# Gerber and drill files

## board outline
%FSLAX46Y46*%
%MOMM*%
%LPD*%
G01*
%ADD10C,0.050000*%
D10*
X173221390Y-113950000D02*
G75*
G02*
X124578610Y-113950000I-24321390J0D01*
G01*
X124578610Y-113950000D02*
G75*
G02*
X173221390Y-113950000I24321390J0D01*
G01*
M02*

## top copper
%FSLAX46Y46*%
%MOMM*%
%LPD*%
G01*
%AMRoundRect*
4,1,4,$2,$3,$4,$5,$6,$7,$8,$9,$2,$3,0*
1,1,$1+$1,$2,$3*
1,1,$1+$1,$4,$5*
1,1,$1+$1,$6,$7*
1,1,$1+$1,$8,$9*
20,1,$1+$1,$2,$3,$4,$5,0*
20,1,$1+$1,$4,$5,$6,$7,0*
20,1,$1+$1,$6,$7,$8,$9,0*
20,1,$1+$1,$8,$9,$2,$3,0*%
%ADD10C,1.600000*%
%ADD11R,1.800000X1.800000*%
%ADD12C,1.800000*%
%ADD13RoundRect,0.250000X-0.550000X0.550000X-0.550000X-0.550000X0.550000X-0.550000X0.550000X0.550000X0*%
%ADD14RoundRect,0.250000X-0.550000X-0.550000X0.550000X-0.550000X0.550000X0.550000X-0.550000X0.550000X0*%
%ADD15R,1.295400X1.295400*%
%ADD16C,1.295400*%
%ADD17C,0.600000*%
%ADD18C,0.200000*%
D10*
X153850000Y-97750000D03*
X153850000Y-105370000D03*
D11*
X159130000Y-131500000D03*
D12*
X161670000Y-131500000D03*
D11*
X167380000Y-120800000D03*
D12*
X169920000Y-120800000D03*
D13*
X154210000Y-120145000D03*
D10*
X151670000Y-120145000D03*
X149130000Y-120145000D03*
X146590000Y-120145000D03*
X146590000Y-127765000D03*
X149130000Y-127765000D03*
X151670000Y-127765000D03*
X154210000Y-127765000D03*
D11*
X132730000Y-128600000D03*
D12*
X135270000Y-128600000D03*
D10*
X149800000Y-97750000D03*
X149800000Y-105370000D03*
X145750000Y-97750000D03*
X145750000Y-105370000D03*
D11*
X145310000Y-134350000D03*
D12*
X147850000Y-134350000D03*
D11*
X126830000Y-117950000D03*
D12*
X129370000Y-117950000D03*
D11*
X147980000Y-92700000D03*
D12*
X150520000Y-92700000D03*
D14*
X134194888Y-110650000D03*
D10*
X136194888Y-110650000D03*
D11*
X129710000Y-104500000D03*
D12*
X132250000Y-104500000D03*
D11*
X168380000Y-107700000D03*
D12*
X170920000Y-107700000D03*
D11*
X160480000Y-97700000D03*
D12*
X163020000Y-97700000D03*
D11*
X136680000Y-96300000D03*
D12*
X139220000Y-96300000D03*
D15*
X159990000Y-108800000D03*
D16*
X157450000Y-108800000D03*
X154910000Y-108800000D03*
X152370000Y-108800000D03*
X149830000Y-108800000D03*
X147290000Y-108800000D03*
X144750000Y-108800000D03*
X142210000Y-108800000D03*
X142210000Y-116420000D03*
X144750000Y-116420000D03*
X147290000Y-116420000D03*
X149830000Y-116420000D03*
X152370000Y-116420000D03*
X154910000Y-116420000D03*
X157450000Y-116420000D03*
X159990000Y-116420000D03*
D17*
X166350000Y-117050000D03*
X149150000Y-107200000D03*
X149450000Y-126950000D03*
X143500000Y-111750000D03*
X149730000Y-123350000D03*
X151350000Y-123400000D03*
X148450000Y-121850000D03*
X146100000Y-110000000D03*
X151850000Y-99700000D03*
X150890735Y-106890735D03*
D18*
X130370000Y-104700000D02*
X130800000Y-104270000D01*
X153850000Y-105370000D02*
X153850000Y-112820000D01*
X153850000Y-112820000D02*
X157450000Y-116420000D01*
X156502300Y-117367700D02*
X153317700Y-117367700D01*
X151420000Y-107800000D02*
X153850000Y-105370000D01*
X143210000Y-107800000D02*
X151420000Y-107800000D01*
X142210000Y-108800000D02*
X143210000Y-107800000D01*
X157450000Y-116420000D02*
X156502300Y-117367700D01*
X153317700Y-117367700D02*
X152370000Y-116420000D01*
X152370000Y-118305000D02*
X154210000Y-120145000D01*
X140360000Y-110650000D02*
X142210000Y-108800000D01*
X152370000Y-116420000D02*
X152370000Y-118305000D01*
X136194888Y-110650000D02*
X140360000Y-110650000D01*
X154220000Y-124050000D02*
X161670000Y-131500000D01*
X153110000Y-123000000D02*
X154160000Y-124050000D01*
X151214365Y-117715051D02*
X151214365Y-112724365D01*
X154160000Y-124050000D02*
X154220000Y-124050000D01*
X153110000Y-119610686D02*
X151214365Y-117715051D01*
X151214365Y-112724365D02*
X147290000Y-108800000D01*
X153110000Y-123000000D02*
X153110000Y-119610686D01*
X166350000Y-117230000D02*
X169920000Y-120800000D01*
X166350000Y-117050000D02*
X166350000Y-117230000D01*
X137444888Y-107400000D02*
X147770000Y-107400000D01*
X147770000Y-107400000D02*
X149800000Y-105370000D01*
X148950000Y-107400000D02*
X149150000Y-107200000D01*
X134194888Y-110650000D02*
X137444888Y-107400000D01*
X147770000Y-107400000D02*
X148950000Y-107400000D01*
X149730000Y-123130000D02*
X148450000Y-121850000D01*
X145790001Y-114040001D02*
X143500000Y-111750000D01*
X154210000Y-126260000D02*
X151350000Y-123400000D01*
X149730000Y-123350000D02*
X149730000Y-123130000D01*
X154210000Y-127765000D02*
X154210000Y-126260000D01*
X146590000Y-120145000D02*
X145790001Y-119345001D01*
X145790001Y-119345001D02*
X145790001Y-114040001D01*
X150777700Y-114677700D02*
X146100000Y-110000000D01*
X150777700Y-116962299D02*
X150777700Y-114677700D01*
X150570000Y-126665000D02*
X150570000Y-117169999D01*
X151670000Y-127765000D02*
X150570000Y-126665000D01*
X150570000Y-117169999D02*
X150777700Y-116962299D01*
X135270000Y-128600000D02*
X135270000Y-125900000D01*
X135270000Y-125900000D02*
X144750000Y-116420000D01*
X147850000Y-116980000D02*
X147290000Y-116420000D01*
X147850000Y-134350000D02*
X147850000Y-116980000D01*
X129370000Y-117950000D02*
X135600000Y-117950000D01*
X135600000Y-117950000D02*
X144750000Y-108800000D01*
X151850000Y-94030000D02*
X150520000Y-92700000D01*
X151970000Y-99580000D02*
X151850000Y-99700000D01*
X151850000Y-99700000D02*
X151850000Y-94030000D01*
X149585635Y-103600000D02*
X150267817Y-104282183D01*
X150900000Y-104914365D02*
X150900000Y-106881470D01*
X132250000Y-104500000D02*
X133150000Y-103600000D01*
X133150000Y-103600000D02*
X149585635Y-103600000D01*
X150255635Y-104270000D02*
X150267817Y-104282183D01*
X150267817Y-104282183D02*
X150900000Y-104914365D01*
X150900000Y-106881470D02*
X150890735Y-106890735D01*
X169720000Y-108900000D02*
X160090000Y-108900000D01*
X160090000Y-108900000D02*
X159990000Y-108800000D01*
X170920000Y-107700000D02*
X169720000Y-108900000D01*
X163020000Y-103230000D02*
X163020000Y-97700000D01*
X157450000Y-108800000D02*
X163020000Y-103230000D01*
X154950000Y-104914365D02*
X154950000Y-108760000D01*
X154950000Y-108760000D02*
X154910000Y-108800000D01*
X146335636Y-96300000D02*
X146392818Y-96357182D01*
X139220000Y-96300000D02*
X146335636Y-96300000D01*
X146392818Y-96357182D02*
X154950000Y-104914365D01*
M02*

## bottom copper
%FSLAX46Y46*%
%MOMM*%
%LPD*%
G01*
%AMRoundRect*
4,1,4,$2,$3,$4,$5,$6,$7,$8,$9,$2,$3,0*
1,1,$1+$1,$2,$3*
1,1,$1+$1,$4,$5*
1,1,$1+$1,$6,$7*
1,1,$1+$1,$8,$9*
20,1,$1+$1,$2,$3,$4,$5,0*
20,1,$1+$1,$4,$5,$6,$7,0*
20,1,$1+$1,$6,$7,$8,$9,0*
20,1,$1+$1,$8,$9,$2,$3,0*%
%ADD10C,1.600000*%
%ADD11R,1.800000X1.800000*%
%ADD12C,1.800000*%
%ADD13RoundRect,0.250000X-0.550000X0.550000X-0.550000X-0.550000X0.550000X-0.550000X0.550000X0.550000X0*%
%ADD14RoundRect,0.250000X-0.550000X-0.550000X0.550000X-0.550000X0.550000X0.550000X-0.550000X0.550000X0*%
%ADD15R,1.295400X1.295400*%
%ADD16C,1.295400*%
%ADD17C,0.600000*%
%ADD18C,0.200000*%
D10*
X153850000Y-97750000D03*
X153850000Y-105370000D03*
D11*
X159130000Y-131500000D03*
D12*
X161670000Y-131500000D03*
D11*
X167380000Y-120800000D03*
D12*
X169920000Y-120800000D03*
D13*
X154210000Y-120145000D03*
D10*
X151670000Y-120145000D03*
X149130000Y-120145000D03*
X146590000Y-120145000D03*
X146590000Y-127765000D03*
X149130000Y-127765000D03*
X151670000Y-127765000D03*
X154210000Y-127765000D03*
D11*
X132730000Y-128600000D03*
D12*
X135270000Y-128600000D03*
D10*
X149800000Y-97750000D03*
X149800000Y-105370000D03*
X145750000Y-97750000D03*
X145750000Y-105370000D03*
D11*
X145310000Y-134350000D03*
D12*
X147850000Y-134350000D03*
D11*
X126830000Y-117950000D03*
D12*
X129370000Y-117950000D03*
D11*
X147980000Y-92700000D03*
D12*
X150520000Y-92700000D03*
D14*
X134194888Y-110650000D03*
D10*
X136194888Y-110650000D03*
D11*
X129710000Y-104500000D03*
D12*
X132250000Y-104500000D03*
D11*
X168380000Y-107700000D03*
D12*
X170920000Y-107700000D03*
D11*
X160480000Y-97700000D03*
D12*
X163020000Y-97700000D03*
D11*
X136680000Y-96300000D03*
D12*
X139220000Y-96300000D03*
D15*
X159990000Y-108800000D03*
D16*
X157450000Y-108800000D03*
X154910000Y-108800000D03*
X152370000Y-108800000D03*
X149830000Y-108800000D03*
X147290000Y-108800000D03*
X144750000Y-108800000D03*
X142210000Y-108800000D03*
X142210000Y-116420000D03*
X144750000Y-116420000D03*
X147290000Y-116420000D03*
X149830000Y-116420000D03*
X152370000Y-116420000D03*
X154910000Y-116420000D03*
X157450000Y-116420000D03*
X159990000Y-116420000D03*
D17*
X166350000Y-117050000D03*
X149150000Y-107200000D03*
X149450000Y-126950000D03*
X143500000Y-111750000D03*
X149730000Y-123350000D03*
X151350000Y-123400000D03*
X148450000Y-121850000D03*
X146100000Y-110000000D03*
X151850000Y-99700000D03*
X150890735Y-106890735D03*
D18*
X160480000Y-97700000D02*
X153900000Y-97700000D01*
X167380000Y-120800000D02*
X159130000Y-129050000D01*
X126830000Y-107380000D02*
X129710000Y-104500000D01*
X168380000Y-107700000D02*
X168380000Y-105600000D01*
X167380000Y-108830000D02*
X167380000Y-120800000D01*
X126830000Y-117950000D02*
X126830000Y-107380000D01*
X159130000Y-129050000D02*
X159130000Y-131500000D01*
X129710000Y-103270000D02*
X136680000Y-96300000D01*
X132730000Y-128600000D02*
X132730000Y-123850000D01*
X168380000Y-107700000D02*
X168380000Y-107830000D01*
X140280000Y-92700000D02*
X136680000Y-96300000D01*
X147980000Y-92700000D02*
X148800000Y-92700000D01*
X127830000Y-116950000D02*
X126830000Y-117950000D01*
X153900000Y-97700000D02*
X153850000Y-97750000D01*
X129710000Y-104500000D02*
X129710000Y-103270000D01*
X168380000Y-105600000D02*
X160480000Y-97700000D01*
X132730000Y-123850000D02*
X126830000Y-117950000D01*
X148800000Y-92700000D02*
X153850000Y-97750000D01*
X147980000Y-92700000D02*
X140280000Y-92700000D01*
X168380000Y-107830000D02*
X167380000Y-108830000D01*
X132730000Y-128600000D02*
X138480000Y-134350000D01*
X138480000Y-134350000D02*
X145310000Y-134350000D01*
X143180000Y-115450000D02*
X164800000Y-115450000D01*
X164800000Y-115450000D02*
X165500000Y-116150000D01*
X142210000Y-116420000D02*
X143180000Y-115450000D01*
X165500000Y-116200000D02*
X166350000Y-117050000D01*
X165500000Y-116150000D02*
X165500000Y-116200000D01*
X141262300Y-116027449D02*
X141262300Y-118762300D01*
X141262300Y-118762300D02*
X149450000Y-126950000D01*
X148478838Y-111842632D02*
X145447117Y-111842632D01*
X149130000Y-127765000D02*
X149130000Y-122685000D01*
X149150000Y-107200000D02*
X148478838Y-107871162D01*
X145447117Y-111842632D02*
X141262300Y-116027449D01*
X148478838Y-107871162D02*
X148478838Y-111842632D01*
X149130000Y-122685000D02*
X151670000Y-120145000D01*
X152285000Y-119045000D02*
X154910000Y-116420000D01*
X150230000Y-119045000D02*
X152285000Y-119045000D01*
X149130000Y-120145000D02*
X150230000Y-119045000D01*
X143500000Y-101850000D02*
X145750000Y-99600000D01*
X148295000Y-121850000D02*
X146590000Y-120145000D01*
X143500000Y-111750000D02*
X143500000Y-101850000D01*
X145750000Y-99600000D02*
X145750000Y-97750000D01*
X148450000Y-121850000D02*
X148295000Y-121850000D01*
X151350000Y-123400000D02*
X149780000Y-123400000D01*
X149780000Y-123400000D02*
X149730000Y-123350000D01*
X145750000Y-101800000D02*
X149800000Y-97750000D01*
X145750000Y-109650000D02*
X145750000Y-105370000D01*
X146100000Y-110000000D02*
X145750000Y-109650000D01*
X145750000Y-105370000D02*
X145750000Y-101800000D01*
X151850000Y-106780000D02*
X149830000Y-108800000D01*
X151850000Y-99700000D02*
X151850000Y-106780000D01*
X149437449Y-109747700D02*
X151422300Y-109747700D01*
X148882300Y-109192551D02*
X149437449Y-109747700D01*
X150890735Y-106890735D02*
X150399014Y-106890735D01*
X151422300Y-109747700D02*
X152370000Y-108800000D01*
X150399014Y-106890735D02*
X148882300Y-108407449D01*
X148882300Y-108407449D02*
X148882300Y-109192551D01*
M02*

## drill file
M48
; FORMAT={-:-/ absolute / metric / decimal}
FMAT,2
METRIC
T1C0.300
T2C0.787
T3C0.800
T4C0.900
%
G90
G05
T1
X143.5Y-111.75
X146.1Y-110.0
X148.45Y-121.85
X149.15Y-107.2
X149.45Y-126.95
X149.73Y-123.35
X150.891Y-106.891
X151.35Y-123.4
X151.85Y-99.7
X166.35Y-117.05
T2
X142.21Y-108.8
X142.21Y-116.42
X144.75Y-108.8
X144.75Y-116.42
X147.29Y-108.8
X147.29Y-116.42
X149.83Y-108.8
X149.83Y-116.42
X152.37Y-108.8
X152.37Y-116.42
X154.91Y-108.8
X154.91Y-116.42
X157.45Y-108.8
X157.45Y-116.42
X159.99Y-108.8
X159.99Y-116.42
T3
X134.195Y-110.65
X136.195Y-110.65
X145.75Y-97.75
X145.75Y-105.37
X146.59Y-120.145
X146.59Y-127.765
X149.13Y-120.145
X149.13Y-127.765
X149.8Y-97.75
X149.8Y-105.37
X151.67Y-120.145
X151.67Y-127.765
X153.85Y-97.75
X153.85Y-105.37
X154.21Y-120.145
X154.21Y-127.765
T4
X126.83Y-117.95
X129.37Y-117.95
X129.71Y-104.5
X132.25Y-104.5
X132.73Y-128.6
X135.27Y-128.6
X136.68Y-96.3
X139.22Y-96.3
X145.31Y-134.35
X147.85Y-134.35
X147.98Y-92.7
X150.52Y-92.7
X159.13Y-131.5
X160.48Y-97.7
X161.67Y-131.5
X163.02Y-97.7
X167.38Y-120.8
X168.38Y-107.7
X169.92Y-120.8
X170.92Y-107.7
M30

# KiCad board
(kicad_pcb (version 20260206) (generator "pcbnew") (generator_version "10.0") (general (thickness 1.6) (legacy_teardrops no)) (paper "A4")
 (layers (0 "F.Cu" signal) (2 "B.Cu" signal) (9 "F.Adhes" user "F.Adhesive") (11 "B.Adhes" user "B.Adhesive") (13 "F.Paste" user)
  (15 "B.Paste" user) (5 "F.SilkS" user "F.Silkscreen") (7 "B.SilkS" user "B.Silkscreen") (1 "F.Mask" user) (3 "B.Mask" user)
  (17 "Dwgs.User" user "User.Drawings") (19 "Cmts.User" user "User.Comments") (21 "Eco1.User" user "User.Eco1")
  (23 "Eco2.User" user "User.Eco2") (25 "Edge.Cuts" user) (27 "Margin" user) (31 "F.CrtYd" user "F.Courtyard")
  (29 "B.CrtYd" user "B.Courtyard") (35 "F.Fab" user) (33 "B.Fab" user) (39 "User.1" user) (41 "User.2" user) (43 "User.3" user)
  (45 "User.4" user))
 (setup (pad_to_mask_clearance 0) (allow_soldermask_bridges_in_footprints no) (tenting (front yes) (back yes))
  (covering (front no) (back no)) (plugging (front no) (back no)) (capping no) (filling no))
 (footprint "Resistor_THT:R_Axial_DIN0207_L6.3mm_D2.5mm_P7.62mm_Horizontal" (layer "F.Cu") (at 153.85 97.75 -90)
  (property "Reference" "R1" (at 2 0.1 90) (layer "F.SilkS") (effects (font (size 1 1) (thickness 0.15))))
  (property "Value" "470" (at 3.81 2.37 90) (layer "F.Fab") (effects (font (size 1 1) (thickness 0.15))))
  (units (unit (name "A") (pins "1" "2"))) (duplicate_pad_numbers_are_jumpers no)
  (pad "1" thru_hole circle (at 0 0 270) (size 1.6 1.6) (drill 0.8) (layers "*.Cu" "*.Mask") (remove_unused_layers no) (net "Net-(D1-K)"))
  (pad "2" thru_hole circle (at 7.62 0 270) (size 1.6 1.6) (drill 0.8) (layers "*.Cu" "*.Mask") (remove_unused_layers no) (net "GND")))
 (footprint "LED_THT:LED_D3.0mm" (layer "F.Cu") (at 159.13 131.5)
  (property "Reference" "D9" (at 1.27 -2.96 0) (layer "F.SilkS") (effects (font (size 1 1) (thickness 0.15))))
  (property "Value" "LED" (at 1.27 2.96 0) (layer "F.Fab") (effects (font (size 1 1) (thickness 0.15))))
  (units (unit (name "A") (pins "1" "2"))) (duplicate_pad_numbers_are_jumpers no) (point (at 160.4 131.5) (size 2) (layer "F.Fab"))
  (pad "1" thru_hole rect (at 0 0) (size 1.8 1.8) (drill 0.9) (layers "*.Cu" "*.Mask") (remove_unused_layers no) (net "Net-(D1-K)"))
  (pad "2" thru_hole circle (at 2.54 0) (size 1.8 1.8) (drill 0.9) (layers "*.Cu" "*.Mask") (remove_unused_layers no) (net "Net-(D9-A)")))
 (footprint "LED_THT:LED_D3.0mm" (layer "F.Cu") (at 167.38 120.8)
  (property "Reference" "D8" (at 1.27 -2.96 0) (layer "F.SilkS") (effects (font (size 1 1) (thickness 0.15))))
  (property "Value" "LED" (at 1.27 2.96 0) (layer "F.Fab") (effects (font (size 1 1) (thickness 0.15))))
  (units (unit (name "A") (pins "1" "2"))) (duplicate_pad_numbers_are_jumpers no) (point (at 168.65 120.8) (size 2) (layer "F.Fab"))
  (pad "1" thru_hole rect (at 0 0) (size 1.8 1.8) (drill 0.9) (layers "*.Cu" "*.Mask") (remove_unused_layers no) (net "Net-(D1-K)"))
  (pad "2" thru_hole circle (at 2.54 0) (size 1.8 1.8) (drill 0.9) (layers "*.Cu" "*.Mask") (remove_unused_layers no) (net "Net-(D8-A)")))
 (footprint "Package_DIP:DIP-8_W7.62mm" (layer "F.Cu") (at 154.21 120.145 -90)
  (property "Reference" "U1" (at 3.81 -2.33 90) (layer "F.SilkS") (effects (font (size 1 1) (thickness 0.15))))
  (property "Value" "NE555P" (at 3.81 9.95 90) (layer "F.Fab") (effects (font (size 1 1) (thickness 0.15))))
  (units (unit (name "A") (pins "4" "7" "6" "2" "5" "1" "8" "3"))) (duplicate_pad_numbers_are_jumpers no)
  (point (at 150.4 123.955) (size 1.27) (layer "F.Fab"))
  (pad "1" thru_hole roundrect (at 0 0 270) (size 1.6 1.6) (drill 0.8) (layers "*.Cu" "*.Mask") (remove_unused_layers no)
   (roundrect_rratio 0.15625) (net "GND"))
  (pad "2" thru_hole circle (at 0 2.54 270) (size 1.6 1.6) (drill 0.8) (layers "*.Cu" "*.Mask") (remove_unused_layers no) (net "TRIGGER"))
  (pad "3" thru_hole circle (at 0 5.08 270) (size 1.6 1.6) (drill 0.8) (layers "*.Cu" "*.Mask") (remove_unused_layers no) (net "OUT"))
  (pad "4" thru_hole circle (at 0 7.62 270) (size 1.6 1.6) (drill 0.8) (layers "*.Cu" "*.Mask") (remove_unused_layers no) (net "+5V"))
  (pad "5" thru_hole circle (at 7.62 7.62 270) (size 1.6 1.6) (drill 0.8) (layers "*.Cu" "*.Mask") (remove_unused_layers no)
   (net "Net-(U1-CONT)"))
  (pad "6" thru_hole circle (at 7.62 5.08 270) (size 1.6 1.6) (drill 0.8) (layers "*.Cu" "*.Mask") (remove_unused_layers no) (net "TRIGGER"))
  (pad "7" thru_hole circle (at 7.62 2.54 270) (size 1.6 1.6) (drill 0.8) (layers "*.Cu" "*.Mask") (remove_unused_layers no)
   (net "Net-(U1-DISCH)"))
  (pad "8" thru_hole circle (at 7.62 0 270) (size 1.6 1.6) (drill 0.8) (layers "*.Cu" "*.Mask") (remove_unused_layers no) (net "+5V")))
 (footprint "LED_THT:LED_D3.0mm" (layer "F.Cu") (at 132.73 128.6)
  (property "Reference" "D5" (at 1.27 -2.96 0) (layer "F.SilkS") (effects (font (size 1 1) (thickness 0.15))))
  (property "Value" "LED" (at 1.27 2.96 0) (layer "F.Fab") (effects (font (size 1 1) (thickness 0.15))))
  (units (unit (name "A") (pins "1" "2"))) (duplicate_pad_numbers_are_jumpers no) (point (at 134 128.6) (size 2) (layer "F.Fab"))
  (pad "1" thru_hole rect (at 0 0) (size 1.8 1.8) (drill 0.9) (layers "*.Cu" "*.Mask") (remove_unused_layers no) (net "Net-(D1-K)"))
  (pad "2" thru_hole circle (at 2.54 0) (size 1.8 1.8) (drill 0.9) (layers "*.Cu" "*.Mask") (remove_unused_layers no) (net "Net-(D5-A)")))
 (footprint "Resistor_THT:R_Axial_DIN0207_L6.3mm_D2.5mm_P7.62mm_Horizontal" (layer "F.Cu") (at 149.8 97.75 -90)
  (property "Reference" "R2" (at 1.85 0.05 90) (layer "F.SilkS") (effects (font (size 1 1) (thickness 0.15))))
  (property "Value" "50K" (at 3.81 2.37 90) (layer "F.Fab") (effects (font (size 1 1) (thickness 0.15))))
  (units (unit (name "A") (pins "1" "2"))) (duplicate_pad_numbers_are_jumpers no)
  (pad "1" thru_hole circle (at 0 0 270) (size 1.6 1.6) (drill 0.8) (layers "*.Cu" "*.Mask") (remove_unused_layers no)
   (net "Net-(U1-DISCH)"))
  (pad "2" thru_hole circle (at 7.62 0 270) (size 1.6 1.6) (drill 0.8) (layers "*.Cu" "*.Mask") (remove_unused_layers no) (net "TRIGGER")))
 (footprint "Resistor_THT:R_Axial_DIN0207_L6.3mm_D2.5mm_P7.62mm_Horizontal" (layer "F.Cu") (at 145.75 97.75 -90)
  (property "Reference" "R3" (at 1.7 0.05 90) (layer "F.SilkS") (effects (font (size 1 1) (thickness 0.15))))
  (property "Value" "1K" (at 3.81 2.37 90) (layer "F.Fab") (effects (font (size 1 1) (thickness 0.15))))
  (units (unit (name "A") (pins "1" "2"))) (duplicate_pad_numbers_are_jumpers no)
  (pad "1" thru_hole circle (at 0 0 270) (size 1.6 1.6) (drill 0.8) (layers "*.Cu" "*.Mask") (remove_unused_layers no) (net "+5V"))
  (pad "2" thru_hole circle (at 7.62 0 270) (size 1.6 1.6) (drill 0.8) (layers "*.Cu" "*.Mask") (remove_unused_layers no)
   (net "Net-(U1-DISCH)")))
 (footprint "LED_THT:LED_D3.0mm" (layer "F.Cu") (at 145.31 134.35)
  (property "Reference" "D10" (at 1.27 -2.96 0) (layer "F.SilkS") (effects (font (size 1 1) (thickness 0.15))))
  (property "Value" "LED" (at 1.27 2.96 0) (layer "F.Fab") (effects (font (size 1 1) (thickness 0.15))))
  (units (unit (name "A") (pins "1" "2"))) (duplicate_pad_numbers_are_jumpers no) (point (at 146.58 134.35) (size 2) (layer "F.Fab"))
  (pad "1" thru_hole rect (at 0 0) (size 1.8 1.8) (drill 0.9) (layers "*.Cu" "*.Mask") (remove_unused_layers no) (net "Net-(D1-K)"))
  (pad "2" thru_hole circle (at 2.54 0) (size 1.8 1.8) (drill 0.9) (layers "*.Cu" "*.Mask") (remove_unused_layers no) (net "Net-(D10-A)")))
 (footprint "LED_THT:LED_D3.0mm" (layer "F.Cu") (at 126.83 117.95)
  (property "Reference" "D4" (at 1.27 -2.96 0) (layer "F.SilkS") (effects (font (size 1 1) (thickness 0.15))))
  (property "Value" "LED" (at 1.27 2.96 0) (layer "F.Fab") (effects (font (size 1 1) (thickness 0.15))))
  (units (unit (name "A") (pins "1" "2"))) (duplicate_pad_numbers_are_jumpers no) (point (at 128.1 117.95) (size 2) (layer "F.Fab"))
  (pad "1" thru_hole rect (at 0 0) (size 1.8 1.8) (drill 0.9) (layers "*.Cu" "*.Mask") (remove_unused_layers no) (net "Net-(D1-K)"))
  (pad "2" thru_hole circle (at 2.54 0) (size 1.8 1.8) (drill 0.9) (layers "*.Cu" "*.Mask") (remove_unused_layers no) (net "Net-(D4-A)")))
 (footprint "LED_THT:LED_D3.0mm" (layer "F.Cu") (at 147.98 92.7)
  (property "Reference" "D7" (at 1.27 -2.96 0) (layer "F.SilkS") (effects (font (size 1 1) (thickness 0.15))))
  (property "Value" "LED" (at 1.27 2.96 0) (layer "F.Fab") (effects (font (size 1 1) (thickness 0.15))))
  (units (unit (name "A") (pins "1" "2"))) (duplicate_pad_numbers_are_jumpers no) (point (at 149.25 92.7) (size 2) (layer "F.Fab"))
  (pad "1" thru_hole rect (at 0 0) (size 1.8 1.8) (drill 0.9) (layers "*.Cu" "*.Mask") (remove_unused_layers no) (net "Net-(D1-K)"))
  (pad "2" thru_hole circle (at 2.54 0) (size 1.8 1.8) (drill 0.9) (layers "*.Cu" "*.Mask") (remove_unused_layers no) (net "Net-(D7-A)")))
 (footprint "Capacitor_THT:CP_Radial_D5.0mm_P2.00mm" (layer "F.Cu") (at 134.194888 110.65)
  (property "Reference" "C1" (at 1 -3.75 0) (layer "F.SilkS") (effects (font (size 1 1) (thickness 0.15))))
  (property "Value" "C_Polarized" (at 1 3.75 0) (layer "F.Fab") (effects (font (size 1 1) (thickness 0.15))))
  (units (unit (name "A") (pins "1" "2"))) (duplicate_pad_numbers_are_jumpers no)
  (pad "1" thru_hole roundrect (at 0 0) (size 1.6 1.6) (drill 0.8) (layers "*.Cu" "*.Mask") (remove_unused_layers no)
   (roundrect_rratio 0.15625) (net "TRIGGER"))
  (pad "2" thru_hole circle (at 2 0) (size 1.6 1.6) (drill 0.8) (layers "*.Cu" "*.Mask") (remove_unused_layers no) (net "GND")))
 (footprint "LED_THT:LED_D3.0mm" (layer "F.Cu") (at 129.71 104.5)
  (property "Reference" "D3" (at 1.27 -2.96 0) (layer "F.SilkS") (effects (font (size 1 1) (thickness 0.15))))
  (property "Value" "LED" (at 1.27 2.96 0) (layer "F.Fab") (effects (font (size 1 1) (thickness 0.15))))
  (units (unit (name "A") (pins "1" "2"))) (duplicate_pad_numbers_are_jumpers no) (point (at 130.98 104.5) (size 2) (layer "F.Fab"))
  (pad "1" thru_hole rect (at 0 0) (size 1.8 1.8) (drill 0.9) (layers "*.Cu" "*.Mask") (remove_unused_layers no) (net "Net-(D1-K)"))
  (pad "2" thru_hole circle (at 2.54 0) (size 1.8 1.8) (drill 0.9) (layers "*.Cu" "*.Mask") (remove_unused_layers no) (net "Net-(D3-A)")))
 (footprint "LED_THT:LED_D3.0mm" (layer "F.Cu") (at 168.38 107.7)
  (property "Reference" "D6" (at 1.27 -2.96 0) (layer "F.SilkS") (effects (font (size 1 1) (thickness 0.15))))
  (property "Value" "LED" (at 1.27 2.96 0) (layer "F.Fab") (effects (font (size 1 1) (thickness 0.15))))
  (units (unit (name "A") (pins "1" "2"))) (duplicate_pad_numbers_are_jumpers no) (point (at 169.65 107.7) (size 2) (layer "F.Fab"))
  (pad "1" thru_hole rect (at 0 0) (size 1.8 1.8) (drill 0.9) (layers "*.Cu" "*.Mask") (remove_unused_layers no) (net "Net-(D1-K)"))
  (pad "2" thru_hole circle (at 2.54 0) (size 1.8 1.8) (drill 0.9) (layers "*.Cu" "*.Mask") (remove_unused_layers no) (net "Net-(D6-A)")))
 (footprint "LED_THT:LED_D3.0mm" (layer "F.Cu") (at 160.48 97.7)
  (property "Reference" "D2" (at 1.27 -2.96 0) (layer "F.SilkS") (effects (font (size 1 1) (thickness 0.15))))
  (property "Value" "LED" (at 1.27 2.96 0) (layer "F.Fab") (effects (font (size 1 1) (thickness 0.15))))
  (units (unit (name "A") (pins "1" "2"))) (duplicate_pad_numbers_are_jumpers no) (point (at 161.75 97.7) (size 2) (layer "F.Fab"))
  (pad "1" thru_hole rect (at 0 0) (size 1.8 1.8) (drill 0.9) (layers "*.Cu" "*.Mask") (remove_unused_layers no) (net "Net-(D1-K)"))
  (pad "2" thru_hole circle (at 2.54 0) (size 1.8 1.8) (drill 0.9) (layers "*.Cu" "*.Mask") (remove_unused_layers no) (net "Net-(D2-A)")))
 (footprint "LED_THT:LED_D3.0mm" (layer "F.Cu") (at 136.68 96.3)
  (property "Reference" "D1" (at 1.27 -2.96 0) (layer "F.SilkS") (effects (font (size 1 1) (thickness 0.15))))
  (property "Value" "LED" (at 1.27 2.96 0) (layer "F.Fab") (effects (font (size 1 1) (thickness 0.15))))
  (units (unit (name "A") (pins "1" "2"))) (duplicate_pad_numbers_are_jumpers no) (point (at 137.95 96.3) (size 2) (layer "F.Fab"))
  (pad "1" thru_hole rect (at 0 0) (size 1.8 1.8) (drill 0.9) (layers "*.Cu" "*.Mask") (remove_unused_layers no) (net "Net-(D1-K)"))
  (pad "2" thru_hole circle (at 2.54 0) (size 1.8 1.8) (drill 0.9) (layers "*.Cu" "*.Mask") (remove_unused_layers no) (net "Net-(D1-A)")))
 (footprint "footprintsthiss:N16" (layer "F.Cu") (at 142.21 116.42 -90)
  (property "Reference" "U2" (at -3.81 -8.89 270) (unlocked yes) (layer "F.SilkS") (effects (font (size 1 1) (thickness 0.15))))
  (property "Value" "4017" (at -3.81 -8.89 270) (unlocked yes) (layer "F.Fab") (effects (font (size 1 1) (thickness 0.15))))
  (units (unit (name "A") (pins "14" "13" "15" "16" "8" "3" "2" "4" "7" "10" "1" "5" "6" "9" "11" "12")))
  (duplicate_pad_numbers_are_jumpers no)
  (pad "1" thru_hole rect (at -7.62 -17.78 270) (size 1.2954 1.2954) (drill 0.7874) (layers "*.Cu" "*.Mask") (remove_unused_layers no)
   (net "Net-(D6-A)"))
  (pad "2" thru_hole circle (at -7.62 -15.24 270) (size 1.2954 1.2954) (drill 0.7874) (layers "*.Cu" "*.Mask") (remove_unused_layers no)
   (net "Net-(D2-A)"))
  (pad "3" thru_hole circle (at -7.62 -12.7 270) (size 1.2954 1.2954) (drill 0.7874) (layers "*.Cu" "*.Mask") (remove_unused_layers no)
   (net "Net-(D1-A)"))
  (pad "4" thru_hole circle (at -7.62 -10.16 270) (size 1.2954 1.2954) (drill 0.7874) (layers "*.Cu" "*.Mask") (remove_unused_layers no)
   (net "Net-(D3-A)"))
  (pad "5" thru_hole circle (at -7.62 -7.62 270) (size 1.2954 1.2954) (drill 0.7874) (layers "*.Cu" "*.Mask") (remove_unused_layers no)
   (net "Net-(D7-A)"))
  (pad "6" thru_hole circle (at -7.62 -5.08 270) (size 1.2954 1.2954) (drill 0.7874) (layers "*.Cu" "*.Mask") (remove_unused_layers no)
   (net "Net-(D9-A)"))
  (pad "7" thru_hole circle (at -7.62 -2.54 270) (size 1.2954 1.2954) (drill 0.7874) (layers "*.Cu" "*.Mask") (remove_unused_layers no)
   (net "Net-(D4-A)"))
  (pad "8" thru_hole circle (at -7.62 0 270) (size 1.2954 1.2954) (drill 0.7874) (layers "*.Cu" "*.Mask") (remove_unused_layers no)
   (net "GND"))
  (pad "9" thru_hole circle (at 0 0 270) (size 1.2954 1.2954) (drill 0.7874) (layers "*.Cu" "*.Mask") (remove_unused_layers no)
   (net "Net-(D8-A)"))
  (pad "10" thru_hole circle (at 0 -2.54 270) (size 1.2954 1.2954) (drill 0.7874) (layers "*.Cu" "*.Mask") (remove_unused_layers no)
   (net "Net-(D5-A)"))
  (pad "11" thru_hole circle (at 0 -5.08 270) (size 1.2954 1.2954) (drill 0.7874) (layers "*.Cu" "*.Mask") (remove_unused_layers no)
   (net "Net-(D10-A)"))
  (pad "12" thru_hole circle (at 0 -7.62 270) (size 1.2954 1.2954) (drill 0.7874) (layers "*.Cu" "*.Mask") (remove_unused_layers no)
   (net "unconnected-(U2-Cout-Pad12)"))
  (pad "13" thru_hole circle (at 0 -10.16 270) (size 1.2954 1.2954) (drill 0.7874) (layers "*.Cu" "*.Mask") (remove_unused_layers no)
   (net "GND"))
  (pad "14" thru_hole circle (at 0 -12.7 270) (size 1.2954 1.2954) (drill 0.7874) (layers "*.Cu" "*.Mask") (remove_unused_layers no)
   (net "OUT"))
  (pad "15" thru_hole circle (at 0 -15.24 270) (size 1.2954 1.2954) (drill 0.7874) (layers "*.Cu" "*.Mask") (remove_unused_layers no)
   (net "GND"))
  (pad "16" thru_hole circle (at 0 -17.78 270) (size 1.2954 1.2954) (drill 0.7874) (layers "*.Cu" "*.Mask") (remove_unused_layers no)
   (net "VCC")))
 (gr_circle (center 148.9 113.95) (end 168.2 99.15) (stroke (width 0.05) (type default)) (fill no) (layer "Edge.Cuts"))
 (segment (start 130.37 104.7) (end 130.8 104.27) (width 0.2) (layer "F.Cu") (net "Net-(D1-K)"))
 (segment (start 160.48 97.7) (end 153.9 97.7) (width 0.2) (layer "B.Cu") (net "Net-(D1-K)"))
 (segment (start 167.38 120.8) (end 159.13 129.05) (width 0.2) (layer "B.Cu") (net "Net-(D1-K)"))
 (segment (start 126.83 107.38) (end 129.71 104.5) (width 0.2) (layer "B.Cu") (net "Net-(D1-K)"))
 (segment (start 168.38 107.7) (end 168.38 105.6) (width 0.2) (layer "B.Cu") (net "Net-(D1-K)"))
 (segment (start 167.38 108.83) (end 167.38 120.8) (width 0.2) (layer "B.Cu") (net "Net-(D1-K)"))
 (segment (start 126.83 117.95) (end 126.83 107.38) (width 0.2) (layer "B.Cu") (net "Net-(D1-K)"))
 (segment (start 159.13 129.05) (end 159.13 131.5) (width 0.2) (layer "B.Cu") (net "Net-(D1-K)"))
 (segment (start 129.71 103.27) (end 136.68 96.3) (width 0.2) (layer "B.Cu") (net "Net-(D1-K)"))
 (segment (start 132.73 128.6) (end 132.73 123.85) (width 0.2) (layer "B.Cu") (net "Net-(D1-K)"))
 (segment (start 168.38 107.7) (end 168.38 107.83) (width 0.2) (layer "B.Cu") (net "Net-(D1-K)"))
 (segment (start 140.28 92.7) (end 136.68 96.3) (width 0.2) (layer "B.Cu") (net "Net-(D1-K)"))
 (segment (start 147.98 92.7) (end 148.8 92.7) (width 0.2) (layer "B.Cu") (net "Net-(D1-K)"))
 (segment (start 127.83 116.95) (end 126.83 117.95) (width 0.2) (layer "B.Cu") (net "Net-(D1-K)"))
 (segment (start 153.9 97.7) (end 153.85 97.75) (width 0.2) (layer "B.Cu") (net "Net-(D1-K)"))
 (segment (start 129.71 104.5) (end 129.71 103.27) (width 0.2) (layer "B.Cu") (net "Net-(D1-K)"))
 (segment (start 168.38 105.6) (end 160.48 97.7) (width 0.2) (layer "B.Cu") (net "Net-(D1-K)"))
 (segment (start 132.73 123.85) (end 126.83 117.95) (width 0.2) (layer "B.Cu") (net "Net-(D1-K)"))
 (segment (start 148.8 92.7) (end 153.85 97.75) (width 0.2) (layer "B.Cu") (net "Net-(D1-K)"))
 (segment (start 147.98 92.7) (end 140.28 92.7) (width 0.2) (layer "B.Cu") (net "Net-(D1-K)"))
 (segment (start 168.38 107.83) (end 167.38 108.83) (width 0.2) (layer "B.Cu") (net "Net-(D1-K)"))
 (segment (start 132.73 128.6) (end 138.48 134.35) (width 0.2) (layer "B.Cu") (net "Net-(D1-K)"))
 (segment (start 138.48 134.35) (end 145.31 134.35) (width 0.2) (layer "B.Cu") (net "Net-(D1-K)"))
 (segment (start 153.85 105.37) (end 153.85 112.82) (width 0.2) (layer "F.Cu") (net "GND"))
 (segment (start 153.85 112.82) (end 157.45 116.42) (width 0.2) (layer "F.Cu") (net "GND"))
 (segment (start 156.5023 117.3677) (end 153.3177 117.3677) (width 0.2) (layer "F.Cu") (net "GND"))
 (segment (start 151.42 107.8) (end 153.85 105.37) (width 0.2) (layer "F.Cu") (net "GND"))
 (segment (start 143.21 107.8) (end 151.42 107.8) (width 0.2) (layer "F.Cu") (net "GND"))
 (segment (start 142.21 108.8) (end 143.21 107.8) (width 0.2) (layer "F.Cu") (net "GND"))
 (segment (start 157.45 116.42) (end 156.5023 117.3677) (width 0.2) (layer "F.Cu") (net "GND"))
 (segment (start 153.3177 117.3677) (end 152.37 116.42) (width 0.2) (layer "F.Cu") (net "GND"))
 (segment (start 152.37 118.305) (end 154.21 120.145) (width 0.2) (layer "F.Cu") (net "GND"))
 (segment (start 140.36 110.65) (end 142.21 108.8) (width 0.2) (layer "F.Cu") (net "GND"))
 (segment (start 152.37 116.42) (end 152.37 118.305) (width 0.2) (layer "F.Cu") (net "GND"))
 (segment (start 136.194888 110.65) (end 140.36 110.65) (width 0.2) (layer "F.Cu") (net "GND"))
 (segment (start 154.22 124.05) (end 161.67 131.5) (width 0.2) (layer "F.Cu") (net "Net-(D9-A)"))
 (segment (start 153.11 123) (end 154.16 124.05) (width 0.2) (layer "F.Cu") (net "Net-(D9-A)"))
 (segment (start 151.214365 117.715051) (end 151.214365 112.724365) (width 0.2) (layer "F.Cu") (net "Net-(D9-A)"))
 (segment (start 154.16 124.05) (end 154.22 124.05) (width 0.2) (layer "F.Cu") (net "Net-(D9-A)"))
 (segment (start 153.11 119.610686) (end 151.214365 117.715051) (width 0.2) (layer "F.Cu") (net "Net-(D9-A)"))
 (segment (start 151.214365 112.724365) (end 147.29 108.8) (width 0.2) (layer "F.Cu") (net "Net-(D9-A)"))
 (segment (start 153.11 123) (end 153.11 119.610686) (width 0.2) (layer "F.Cu") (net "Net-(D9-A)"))
 (segment (start 166.35 117.23) (end 169.92 120.8) (width 0.2) (layer "F.Cu") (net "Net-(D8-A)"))
 (segment (start 166.35 117.05) (end 166.35 117.23) (width 0.2) (layer "F.Cu") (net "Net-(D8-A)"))
 (via (at 166.35 117.05) (size 0.6) (drill 0.3) (layers "F.Cu" "B.Cu") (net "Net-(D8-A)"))
 (segment (start 143.18 115.45) (end 164.8 115.45) (width 0.2) (layer "B.Cu") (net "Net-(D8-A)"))
 (segment (start 164.8 115.45) (end 165.5 116.15) (width 0.2) (layer "B.Cu") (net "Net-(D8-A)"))
 (segment (start 142.21 116.42) (end 143.18 115.45) (width 0.2) (layer "B.Cu") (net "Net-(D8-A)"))
 (segment (start 165.5 116.2) (end 166.35 117.05) (width 0.2) (layer "B.Cu") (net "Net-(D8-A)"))
 (segment (start 165.5 116.15) (end 165.5 116.2) (width 0.2) (layer "B.Cu") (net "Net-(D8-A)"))
 (segment (start 137.444888 107.4) (end 147.77 107.4) (width 0.2) (layer "F.Cu") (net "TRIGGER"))
 (segment (start 147.77 107.4) (end 149.8 105.37) (width 0.2) (layer "F.Cu") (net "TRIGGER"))
 (segment (start 148.95 107.4) (end 149.15 107.2) (width 0.2) (layer "F.Cu") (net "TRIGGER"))
 (segment (start 134.194888 110.65) (end 137.444888 107.4) (width 0.2) (layer "F.Cu") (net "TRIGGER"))
 (segment (start 147.77 107.4) (end 148.95 107.4) (width 0.2) (layer "F.Cu") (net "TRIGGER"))
 (via (at 149.15 107.2) (size 0.6) (drill 0.3) (layers "F.Cu" "B.Cu") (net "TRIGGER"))
 (via (at 149.45 126.95) (size 0.6) (drill 0.3) (layers "F.Cu" "B.Cu") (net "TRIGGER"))
 (segment (start 141.2623 116.027449) (end 141.2623 118.7623) (width 0.2) (layer "B.Cu") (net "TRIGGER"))
 (segment (start 141.2623 118.7623) (end 149.45 126.95) (width 0.2) (layer "B.Cu") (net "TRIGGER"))
 (segment (start 148.478838 111.842632) (end 145.447117 111.842632) (width 0.2) (layer "B.Cu") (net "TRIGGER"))
 (segment (start 149.13 127.765) (end 149.13 122.685) (width 0.2) (layer "B.Cu") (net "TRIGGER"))
 (segment (start 149.15 107.2) (end 148.478838 107.871162) (width 0.2) (layer "B.Cu") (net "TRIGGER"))
 (segment (start 145.447117 111.842632) (end 141.2623 116.027449) (width 0.2) (layer "B.Cu") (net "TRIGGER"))
 (segment (start 148.478838 107.871162) (end 148.478838 111.842632) (width 0.2) (layer "B.Cu") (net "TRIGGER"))
 (segment (start 149.13 122.685) (end 151.67 120.145) (width 0.2) (layer "B.Cu") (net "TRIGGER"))
 (segment (start 152.285 119.045) (end 154.91 116.42) (width 0.2) (layer "B.Cu") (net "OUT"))
 (segment (start 150.23 119.045) (end 152.285 119.045) (width 0.2) (layer "B.Cu") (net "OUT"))
 (segment (start 149.13 120.145) (end 150.23 119.045) (width 0.2) (layer "B.Cu") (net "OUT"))
 (segment (start 149.73 123.13) (end 148.45 121.85) (width 0.2) (layer "F.Cu") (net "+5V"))
 (segment (start 145.790001 114.040001) (end 143.5 111.75) (width 0.2) (layer "F.Cu") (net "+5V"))
 (segment (start 154.21 126.26) (end 151.35 123.4) (width 0.2) (layer "F.Cu") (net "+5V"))
 (segment (start 149.73 123.35) (end 149.73 123.13) (width 0.2) (layer "F.Cu") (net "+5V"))
 (segment (start 154.21 127.765) (end 154.21 126.26) (width 0.2) (layer "F.Cu") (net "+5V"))
 (segment (start 146.59 120.145) (end 145.790001 119.345001) (width 0.2) (layer "F.Cu") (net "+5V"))
 (segment (start 145.790001 119.345001) (end 145.790001 114.040001) (width 0.2) (layer "F.Cu") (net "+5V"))
 (via (at 143.5 111.75) (size 0.6) (drill 0.3) (layers "F.Cu" "B.Cu") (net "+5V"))
 (via (at 149.73 123.35) (size 0.6) (drill 0.3) (layers "F.Cu" "B.Cu") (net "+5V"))
 (via (at 151.35 123.4) (size 0.6) (drill 0.3) (layers "F.Cu" "B.Cu") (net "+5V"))
 (via (at 148.45 121.85) (size 0.6) (drill 0.3) (layers "F.Cu" "B.Cu") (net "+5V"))
 (segment (start 143.5 101.85) (end 145.75 99.6) (width 0.2) (layer "B.Cu") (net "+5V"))
 (segment (start 148.295 121.85) (end 146.59 120.145) (width 0.2) (layer "B.Cu") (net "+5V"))
 (segment (start 143.5 111.75) (end 143.5 101.85) (width 0.2) (layer "B.Cu") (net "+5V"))
 (segment (start 145.75 99.6) (end 145.75 97.75) (width 0.2) (layer "B.Cu") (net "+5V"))
 (segment (start 148.45 121.85) (end 148.295 121.85) (width 0.2) (layer "B.Cu") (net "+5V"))
 (segment (start 151.35 123.4) (end 149.78 123.4) (width 0.2) (layer "B.Cu") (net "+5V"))
 (segment (start 149.78 123.4) (end 149.73 123.35) (width 0.2) (layer "B.Cu") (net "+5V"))
 (segment (start 150.7777 114.6777) (end 146.1 110) (width 0.2) (layer "F.Cu") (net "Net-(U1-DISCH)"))
 (segment (start 150.7777 116.962299) (end 150.7777 114.6777) (width 0.2) (layer "F.Cu") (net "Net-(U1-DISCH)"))
 (segment (start 150.57 126.665) (end 150.57 117.169999) (width 0.2) (layer "F.Cu") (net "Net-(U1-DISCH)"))
 (segment (start 151.67 127.765) (end 150.57 126.665) (width 0.2) (layer "F.Cu") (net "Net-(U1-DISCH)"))
 (segment (start 150.57 117.169999) (end 150.7777 116.962299) (width 0.2) (layer "F.Cu") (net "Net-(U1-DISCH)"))
 (via (at 146.1 110) (size 0.6) (drill 0.3) (layers "F.Cu" "B.Cu") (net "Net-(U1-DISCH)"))
 (segment (start 145.75 101.8) (end 149.8 97.75) (width 0.2) (layer "B.Cu") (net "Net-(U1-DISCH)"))
 (segment (start 145.75 109.65) (end 145.75 105.37) (width 0.2) (layer "B.Cu") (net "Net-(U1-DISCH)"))
 (segment (start 146.1 110) (end 145.75 109.65) (width 0.2) (layer "B.Cu") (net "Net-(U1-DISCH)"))
 (segment (start 145.75 105.37) (end 145.75 101.8) (width 0.2) (layer "B.Cu") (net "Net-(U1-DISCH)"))
 (segment (start 135.27 128.6) (end 135.27 125.9) (width 0.2) (layer "F.Cu") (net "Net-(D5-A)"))
 (segment (start 135.27 125.9) (end 144.75 116.42) (width 0.2) (layer "F.Cu") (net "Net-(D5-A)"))
 (segment (start 147.85 116.98) (end 147.29 116.42) (width 0.2) (layer "F.Cu") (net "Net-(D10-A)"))
 (segment (start 147.85 134.35) (end 147.85 116.98) (width 0.2) (layer "F.Cu") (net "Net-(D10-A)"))
 (segment (start 129.37 117.95) (end 135.6 117.95) (width 0.2) (layer "F.Cu") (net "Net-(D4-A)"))
 (segment (start 135.6 117.95) (end 144.75 108.8) (width 0.2) (layer "F.Cu") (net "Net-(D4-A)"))
 (segment (start 151.85 94.03) (end 150.52 92.7) (width 0.2) (layer "F.Cu") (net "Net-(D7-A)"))
 (segment (start 151.97 99.58) (end 151.85 99.7) (width 0.2) (layer "F.Cu") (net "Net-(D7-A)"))
 (segment (start 151.85 99.7) (end 151.85 94.03) (width 0.2) (layer "F.Cu") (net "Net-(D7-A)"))
 (via (at 151.85 99.7) (size 0.6) (drill 0.3) (layers "F.Cu" "B.Cu") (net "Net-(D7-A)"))
 (segment (start 151.85 106.78) (end 149.83 108.8) (width 0.2) (layer "B.Cu") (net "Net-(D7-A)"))
 (segment (start 151.85 99.7) (end 151.85 106.78) (width 0.2) (layer "B.Cu") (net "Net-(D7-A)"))
 (segment (start 149.585635 103.6) (end 150.267817 104.282183) (width 0.2) (layer "F.Cu") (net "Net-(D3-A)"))
 (segment (start 150.9 104.914365) (end 150.9 106.88147) (width 0.2) (layer "F.Cu") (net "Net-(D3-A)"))
 (segment (start 132.25 104.5) (end 133.15 103.6) (width 0.2) (layer "F.Cu") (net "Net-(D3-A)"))
 (segment (start 133.15 103.6) (end 149.585635 103.6) (width 0.2) (layer "F.Cu") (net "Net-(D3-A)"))
 (segment (start 150.255635 104.27) (end 150.267817 104.282183) (width 0.2) (layer "F.Cu") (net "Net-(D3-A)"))
 (segment (start 150.267817 104.282183) (end 150.9 104.914365) (width 0.2) (layer "F.Cu") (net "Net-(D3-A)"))
 (segment (start 150.9 106.88147) (end 150.890735 106.890735) (width 0.2) (layer "F.Cu") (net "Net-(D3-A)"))
 (via (at 150.890735 106.890735) (size 0.6) (drill 0.3) (layers "F.Cu" "B.Cu") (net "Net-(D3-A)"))
 (segment (start 149.437449 109.7477) (end 151.4223 109.7477) (width 0.2) (layer "B.Cu") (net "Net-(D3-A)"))
 (segment (start 148.8823 109.192551) (end 149.437449 109.7477) (width 0.2) (layer "B.Cu") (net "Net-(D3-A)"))
 (segment (start 150.890735 106.890735) (end 150.399014 106.890735) (width 0.2) (layer "B.Cu") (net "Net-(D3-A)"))
 (segment (start 151.4223 109.7477) (end 152.37 108.8) (width 0.2) (layer "B.Cu") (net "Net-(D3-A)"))
 (segment (start 150.399014 106.890735) (end 148.8823 108.407449) (width 0.2) (layer "B.Cu") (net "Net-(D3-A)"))
 (segment (start 148.8823 108.407449) (end 148.8823 109.192551) (width 0.2) (layer "B.Cu") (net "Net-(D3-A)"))
 (segment (start 169.72 108.9) (end 160.09 108.9) (width 0.2) (layer "F.Cu") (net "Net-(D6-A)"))
 (segment (start 160.09 108.9) (end 159.99 108.8) (width 0.2) (layer "F.Cu") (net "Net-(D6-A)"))
 (segment (start 170.92 107.7) (end 169.72 108.9) (width 0.2) (layer "F.Cu") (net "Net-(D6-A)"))
 (segment (start 163.02 103.23) (end 163.02 97.7) (width 0.2) (layer "F.Cu") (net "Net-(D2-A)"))
 (segment (start 157.45 108.8) (end 163.02 103.23) (width 0.2) (layer "F.Cu") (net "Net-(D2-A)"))
 (segment (start 154.95 104.914365) (end 154.95 108.76) (width 0.2) (layer "F.Cu") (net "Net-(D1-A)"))
 (segment (start 154.95 108.76) (end 154.91 108.8) (width 0.2) (layer "F.Cu") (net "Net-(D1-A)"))
 (segment (start 146.335636 96.3) (end 146.392818 96.357182) (width 0.2) (layer "F.Cu") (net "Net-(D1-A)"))
 (segment (start 139.22 96.3) (end 146.335636 96.3) (width 0.2) (layer "F.Cu") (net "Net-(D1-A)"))
 (segment (start 146.392818 96.357182) (end 154.95 104.914365) (width 0.2) (layer "F.Cu") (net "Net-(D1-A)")))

